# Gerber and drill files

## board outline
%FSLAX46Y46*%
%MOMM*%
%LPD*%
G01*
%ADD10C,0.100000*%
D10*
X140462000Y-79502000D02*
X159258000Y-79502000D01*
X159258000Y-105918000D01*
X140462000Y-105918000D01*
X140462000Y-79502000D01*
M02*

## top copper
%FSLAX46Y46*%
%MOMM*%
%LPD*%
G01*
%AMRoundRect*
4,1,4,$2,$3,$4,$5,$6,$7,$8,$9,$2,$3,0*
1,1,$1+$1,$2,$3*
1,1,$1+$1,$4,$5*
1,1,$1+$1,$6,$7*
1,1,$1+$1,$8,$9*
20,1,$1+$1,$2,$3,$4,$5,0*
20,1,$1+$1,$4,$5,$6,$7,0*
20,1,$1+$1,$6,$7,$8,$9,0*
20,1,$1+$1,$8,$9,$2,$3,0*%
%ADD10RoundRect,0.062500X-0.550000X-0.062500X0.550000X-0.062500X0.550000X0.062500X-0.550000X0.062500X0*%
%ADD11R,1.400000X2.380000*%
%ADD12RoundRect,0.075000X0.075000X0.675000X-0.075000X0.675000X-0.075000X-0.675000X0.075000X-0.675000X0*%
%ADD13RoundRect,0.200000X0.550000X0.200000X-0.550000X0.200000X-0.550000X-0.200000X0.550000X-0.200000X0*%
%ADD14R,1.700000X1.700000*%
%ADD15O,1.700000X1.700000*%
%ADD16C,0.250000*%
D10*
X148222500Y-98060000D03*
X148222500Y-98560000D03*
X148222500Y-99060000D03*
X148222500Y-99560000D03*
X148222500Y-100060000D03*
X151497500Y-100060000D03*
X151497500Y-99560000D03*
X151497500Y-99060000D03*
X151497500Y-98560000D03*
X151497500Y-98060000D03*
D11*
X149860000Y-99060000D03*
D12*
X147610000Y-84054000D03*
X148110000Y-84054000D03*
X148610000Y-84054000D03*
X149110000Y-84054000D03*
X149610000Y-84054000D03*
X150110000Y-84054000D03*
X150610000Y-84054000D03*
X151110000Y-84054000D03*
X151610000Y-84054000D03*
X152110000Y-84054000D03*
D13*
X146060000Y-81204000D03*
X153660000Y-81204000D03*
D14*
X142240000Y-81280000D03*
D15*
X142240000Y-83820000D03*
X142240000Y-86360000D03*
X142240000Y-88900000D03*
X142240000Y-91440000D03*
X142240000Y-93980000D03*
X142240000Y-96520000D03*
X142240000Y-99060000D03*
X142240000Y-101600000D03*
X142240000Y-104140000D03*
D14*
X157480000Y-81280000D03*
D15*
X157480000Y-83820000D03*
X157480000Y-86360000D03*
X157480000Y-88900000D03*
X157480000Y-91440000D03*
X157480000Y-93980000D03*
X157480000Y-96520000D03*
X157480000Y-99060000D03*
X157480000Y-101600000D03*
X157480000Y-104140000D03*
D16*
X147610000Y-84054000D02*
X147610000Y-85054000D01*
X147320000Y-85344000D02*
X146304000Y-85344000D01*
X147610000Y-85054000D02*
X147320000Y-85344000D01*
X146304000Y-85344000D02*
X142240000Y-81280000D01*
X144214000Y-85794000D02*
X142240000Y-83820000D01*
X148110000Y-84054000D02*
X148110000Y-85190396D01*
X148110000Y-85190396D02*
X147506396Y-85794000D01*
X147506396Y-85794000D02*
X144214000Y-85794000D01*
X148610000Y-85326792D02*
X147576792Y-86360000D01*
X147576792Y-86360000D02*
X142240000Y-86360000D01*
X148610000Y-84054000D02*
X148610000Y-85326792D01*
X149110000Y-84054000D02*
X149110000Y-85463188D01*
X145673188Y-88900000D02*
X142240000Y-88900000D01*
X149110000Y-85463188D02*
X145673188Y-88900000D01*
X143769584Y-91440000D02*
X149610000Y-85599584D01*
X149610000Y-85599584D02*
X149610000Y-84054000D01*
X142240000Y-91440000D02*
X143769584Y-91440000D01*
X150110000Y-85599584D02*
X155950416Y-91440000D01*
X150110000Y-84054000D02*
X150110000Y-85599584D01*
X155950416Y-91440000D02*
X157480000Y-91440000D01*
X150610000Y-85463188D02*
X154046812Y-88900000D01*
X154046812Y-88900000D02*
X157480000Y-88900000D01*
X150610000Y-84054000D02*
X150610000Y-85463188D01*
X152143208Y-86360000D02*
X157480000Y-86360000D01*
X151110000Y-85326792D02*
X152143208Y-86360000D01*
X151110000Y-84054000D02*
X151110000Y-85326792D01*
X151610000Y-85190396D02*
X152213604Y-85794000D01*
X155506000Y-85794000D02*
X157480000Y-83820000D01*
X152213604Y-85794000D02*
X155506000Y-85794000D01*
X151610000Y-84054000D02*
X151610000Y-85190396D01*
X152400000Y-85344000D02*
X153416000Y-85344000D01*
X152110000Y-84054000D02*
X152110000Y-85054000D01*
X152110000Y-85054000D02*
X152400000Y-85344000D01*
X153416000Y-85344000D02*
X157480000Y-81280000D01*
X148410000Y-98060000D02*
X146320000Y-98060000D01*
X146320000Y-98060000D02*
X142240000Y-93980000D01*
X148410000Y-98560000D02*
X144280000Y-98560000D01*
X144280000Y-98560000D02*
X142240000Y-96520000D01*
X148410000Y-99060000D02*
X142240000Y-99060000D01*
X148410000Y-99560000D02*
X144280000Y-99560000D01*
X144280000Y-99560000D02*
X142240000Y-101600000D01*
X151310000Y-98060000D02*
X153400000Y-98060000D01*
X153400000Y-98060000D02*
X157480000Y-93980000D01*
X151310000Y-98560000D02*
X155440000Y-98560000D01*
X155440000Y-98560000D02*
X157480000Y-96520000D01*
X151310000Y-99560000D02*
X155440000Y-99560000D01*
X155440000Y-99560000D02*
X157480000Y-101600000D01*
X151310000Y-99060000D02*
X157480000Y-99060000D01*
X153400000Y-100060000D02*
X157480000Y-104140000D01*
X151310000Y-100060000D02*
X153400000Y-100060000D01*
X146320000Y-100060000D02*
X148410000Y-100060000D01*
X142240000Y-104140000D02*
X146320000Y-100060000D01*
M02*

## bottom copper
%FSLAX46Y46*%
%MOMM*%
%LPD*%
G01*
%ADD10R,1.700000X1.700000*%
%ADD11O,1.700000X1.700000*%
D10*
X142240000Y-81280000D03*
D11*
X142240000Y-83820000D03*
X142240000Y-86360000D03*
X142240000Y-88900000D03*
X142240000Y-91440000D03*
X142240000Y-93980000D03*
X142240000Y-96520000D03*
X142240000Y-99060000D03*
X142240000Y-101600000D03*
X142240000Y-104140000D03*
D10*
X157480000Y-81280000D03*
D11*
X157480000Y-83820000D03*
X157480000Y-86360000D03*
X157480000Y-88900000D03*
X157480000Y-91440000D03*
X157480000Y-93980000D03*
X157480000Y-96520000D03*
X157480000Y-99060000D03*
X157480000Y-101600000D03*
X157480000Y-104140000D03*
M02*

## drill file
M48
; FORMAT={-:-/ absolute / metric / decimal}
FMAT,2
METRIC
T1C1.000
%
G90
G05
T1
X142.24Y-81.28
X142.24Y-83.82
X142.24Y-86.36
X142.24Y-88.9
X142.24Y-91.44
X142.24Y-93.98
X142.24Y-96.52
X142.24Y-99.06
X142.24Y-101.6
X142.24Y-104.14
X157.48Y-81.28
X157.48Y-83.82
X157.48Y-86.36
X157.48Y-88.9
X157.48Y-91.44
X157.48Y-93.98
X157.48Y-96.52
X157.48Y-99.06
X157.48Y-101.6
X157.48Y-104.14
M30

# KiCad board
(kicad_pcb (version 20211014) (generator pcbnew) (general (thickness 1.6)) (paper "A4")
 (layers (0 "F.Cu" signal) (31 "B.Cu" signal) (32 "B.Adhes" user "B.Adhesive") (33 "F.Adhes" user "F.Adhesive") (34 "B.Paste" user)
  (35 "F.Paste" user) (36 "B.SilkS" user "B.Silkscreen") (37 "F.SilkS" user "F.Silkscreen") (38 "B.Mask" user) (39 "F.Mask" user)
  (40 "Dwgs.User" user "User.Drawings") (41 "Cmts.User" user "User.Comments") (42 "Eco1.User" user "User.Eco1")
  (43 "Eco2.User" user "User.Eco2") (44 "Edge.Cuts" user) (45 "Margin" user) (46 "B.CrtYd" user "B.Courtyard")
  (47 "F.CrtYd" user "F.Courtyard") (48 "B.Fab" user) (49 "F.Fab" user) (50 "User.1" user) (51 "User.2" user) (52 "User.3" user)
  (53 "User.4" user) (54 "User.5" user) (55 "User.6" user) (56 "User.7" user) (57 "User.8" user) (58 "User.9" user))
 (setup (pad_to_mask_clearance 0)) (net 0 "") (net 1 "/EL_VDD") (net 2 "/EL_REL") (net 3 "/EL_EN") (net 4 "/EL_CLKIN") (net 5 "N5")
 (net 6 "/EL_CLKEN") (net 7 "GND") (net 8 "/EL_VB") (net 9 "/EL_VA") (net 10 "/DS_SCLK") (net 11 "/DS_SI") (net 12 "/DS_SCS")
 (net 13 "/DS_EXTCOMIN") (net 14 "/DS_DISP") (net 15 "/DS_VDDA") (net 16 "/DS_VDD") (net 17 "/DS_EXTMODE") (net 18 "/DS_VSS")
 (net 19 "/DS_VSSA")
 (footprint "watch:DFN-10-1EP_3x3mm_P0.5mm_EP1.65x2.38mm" (layer "F.Cu") (at 149.86 99.06)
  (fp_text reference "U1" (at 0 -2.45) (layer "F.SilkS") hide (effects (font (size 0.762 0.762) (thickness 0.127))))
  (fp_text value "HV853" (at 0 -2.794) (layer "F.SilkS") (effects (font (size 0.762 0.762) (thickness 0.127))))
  (pad "" smd roundrect (at -0.41 0.595) (size 0.67 0.96) (layers "F.Paste") (roundrect_rratio 0.25))
  (pad "" smd roundrect (at 0.41 0.595) (size 0.67 0.96) (layers "F.Paste") (roundrect_rratio 0.25))
  (pad "" smd roundrect (at 0.41 -0.595) (size 0.67 0.96) (layers "F.Paste") (roundrect_rratio 0.25))
  (pad "" smd roundrect (at -0.41 -0.595) (size 0.67 0.96) (layers "F.Paste") (roundrect_rratio 0.25))
  (pad "1" smd roundrect (at -1.6375 -1) (size 1.225 0.25) (layers "F.Cu" "F.Paste" "F.Mask") (roundrect_rratio 0.25) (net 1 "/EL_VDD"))
  (pad "2" smd roundrect (at -1.6375 -0.5) (size 1.225 0.25) (layers "F.Cu" "F.Paste" "F.Mask") (roundrect_rratio 0.25) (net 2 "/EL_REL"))
  (pad "3" smd roundrect (at -1.6375 0) (size 1.225 0.25) (layers "F.Cu" "F.Paste" "F.Mask") (roundrect_rratio 0.25) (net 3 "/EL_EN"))
  (pad "4" smd roundrect (at -1.6375 0.5) (size 1.225 0.25) (layers "F.Cu" "F.Paste" "F.Mask") (roundrect_rratio 0.25) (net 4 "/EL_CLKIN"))
  (pad "5" smd roundrect (at -1.6375 1) (size 1.225 0.25) (layers "F.Cu" "F.Paste" "F.Mask") (roundrect_rratio 0.25) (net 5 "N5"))
  (pad "6" smd roundrect (at 1.6375 1) (size 1.225 0.25) (layers "F.Cu" "F.Paste" "F.Mask") (roundrect_rratio 0.25) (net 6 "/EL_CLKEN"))
  (pad "7" smd roundrect (at 1.6375 0.5) (size 1.225 0.25) (layers "F.Cu" "F.Paste" "F.Mask") (roundrect_rratio 0.25) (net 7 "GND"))
  (pad "8" smd roundrect (at 1.6375 0) (size 1.225 0.25) (layers "F.Cu" "F.Paste" "F.Mask") (roundrect_rratio 0.25) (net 7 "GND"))
  (pad "9" smd roundrect (at 1.6375 -0.5) (size 1.225 0.25) (layers "F.Cu" "F.Paste" "F.Mask") (roundrect_rratio 0.25) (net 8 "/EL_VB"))
  (pad "10" smd roundrect (at 1.6375 -1) (size 1.225 0.25) (layers "F.Cu" "F.Paste" "F.Mask") (roundrect_rratio 0.25) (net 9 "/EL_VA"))
  (pad "11" smd rect (at 0 0) (size 1.4 2.38) (layers "F.Cu" "F.Mask")))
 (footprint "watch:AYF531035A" (layer "F.Cu") (at 149.86 81.204 180)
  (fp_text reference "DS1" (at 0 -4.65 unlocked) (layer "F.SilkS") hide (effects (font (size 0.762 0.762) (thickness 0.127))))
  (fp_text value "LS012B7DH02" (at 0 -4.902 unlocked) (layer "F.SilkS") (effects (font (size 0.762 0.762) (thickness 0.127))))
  (pad "1" smd roundrect (at 2.25 -2.85 180) (size 0.3 1.5) (layers "F.Cu" "F.Paste" "F.Mask") (roundrect_rratio 0.25) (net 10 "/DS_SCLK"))
  (pad "2" smd roundrect (at 1.75 -2.85 180) (size 0.3 1.5) (layers "F.Cu" "F.Paste" "F.Mask") (roundrect_rratio 0.25) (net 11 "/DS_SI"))
  (pad "3" smd roundrect (at 1.25 -2.85 180) (size 0.3 1.5) (layers "F.Cu" "F.Paste" "F.Mask") (roundrect_rratio 0.25) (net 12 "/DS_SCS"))
  (pad "4" smd roundrect (at 0.75 -2.85 180) (size 0.3 1.5) (layers "F.Cu" "F.Paste" "F.Mask") (roundrect_rratio 0.25)
   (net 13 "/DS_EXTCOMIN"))
  (pad "5" smd roundrect (at 0.25 -2.85 180) (size 0.3 1.5) (layers "F.Cu" "F.Paste" "F.Mask") (roundrect_rratio 0.25) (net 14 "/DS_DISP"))
  (pad "6" smd roundrect (at -0.25 -2.85 180) (size 0.3 1.5) (layers "F.Cu" "F.Paste" "F.Mask") (roundrect_rratio 0.25) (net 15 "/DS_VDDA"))
  (pad "7" smd roundrect (at -0.75 -2.85 180) (size 0.3 1.5) (layers "F.Cu" "F.Paste" "F.Mask") (roundrect_rratio 0.25) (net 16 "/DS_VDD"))
  (pad "8" smd roundrect (at -1.25 -2.85 180) (size 0.3 1.5) (layers "F.Cu" "F.Paste" "F.Mask") (roundrect_rratio 0.25)
   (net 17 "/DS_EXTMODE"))
  (pad "9" smd roundrect (at -1.75 -2.85 180) (size 0.3 1.5) (layers "F.Cu" "F.Paste" "F.Mask") (roundrect_rratio 0.25) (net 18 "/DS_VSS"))
  (pad "10" smd roundrect (at -2.25 -2.85 180) (size 0.3 1.5) (layers "F.Cu" "F.Paste" "F.Mask") (roundrect_rratio 0.25) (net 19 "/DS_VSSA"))
  (pad "MT" smd roundrect (at 3.8 0 180) (size 1.5 0.8) (layers "F.Cu" "F.Paste" "F.Mask") (roundrect_rratio 0.25))
  (pad "MT" smd roundrect (at -3.8 0 180) (size 1.5 0.8) (layers "F.Cu" "F.Paste" "F.Mask") (roundrect_rratio 0.25)))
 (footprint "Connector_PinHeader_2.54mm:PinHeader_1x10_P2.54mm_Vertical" (layer "B.Cu") (at 142.24 81.28 180)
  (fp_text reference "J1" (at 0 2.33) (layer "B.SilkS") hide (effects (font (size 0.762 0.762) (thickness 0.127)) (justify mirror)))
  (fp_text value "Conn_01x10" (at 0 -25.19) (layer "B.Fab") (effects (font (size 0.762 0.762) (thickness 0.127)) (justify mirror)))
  (pad "1" thru_hole rect (at 0 0 180) (size 1.7 1.7) (drill 1) (layers *.Cu *.Mask) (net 10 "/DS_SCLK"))
  (pad "2" thru_hole oval (at 0 -2.54 180) (size 1.7 1.7) (drill 1) (layers *.Cu *.Mask) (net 11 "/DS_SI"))
  (pad "3" thru_hole oval (at 0 -5.08 180) (size 1.7 1.7) (drill 1) (layers *.Cu *.Mask) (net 12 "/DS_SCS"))
  (pad "4" thru_hole oval (at 0 -7.62 180) (size 1.7 1.7) (drill 1) (layers *.Cu *.Mask) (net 13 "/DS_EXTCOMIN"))
  (pad "5" thru_hole oval (at 0 -10.16 180) (size 1.7 1.7) (drill 1) (layers *.Cu *.Mask) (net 14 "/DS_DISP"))
  (pad "6" thru_hole oval (at 0 -12.7 180) (size 1.7 1.7) (drill 1) (layers *.Cu *.Mask) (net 1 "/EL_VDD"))
  (pad "7" thru_hole oval (at 0 -15.24 180) (size 1.7 1.7) (drill 1) (layers *.Cu *.Mask) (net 2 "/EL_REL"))
  (pad "8" thru_hole oval (at 0 -17.78 180) (size 1.7 1.7) (drill 1) (layers *.Cu *.Mask) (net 3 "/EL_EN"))
  (pad "9" thru_hole oval (at 0 -20.32 180) (size 1.7 1.7) (drill 1) (layers *.Cu *.Mask) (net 4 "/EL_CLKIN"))
  (pad "10" thru_hole oval (at 0 -22.86 180) (size 1.7 1.7) (drill 1) (layers *.Cu *.Mask) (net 5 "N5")))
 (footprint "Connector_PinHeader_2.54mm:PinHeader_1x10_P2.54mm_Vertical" (layer "B.Cu") (at 157.48 81.28 180)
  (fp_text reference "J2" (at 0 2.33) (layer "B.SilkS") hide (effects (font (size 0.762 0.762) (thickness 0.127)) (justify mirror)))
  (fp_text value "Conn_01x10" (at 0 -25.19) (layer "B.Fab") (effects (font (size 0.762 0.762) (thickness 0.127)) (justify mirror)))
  (pad "1" thru_hole rect (at 0 0 180) (size 1.7 1.7) (drill 1) (layers *.Cu *.Mask) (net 19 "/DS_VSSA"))
  (pad "2" thru_hole oval (at 0 -2.54 180) (size 1.7 1.7) (drill 1) (layers *.Cu *.Mask) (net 18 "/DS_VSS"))
  (pad "3" thru_hole oval (at 0 -5.08 180) (size 1.7 1.7) (drill 1) (layers *.Cu *.Mask) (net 17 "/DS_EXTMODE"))
  (pad "4" thru_hole oval (at 0 -7.62 180) (size 1.7 1.7) (drill 1) (layers *.Cu *.Mask) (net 16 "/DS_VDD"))
  (pad "5" thru_hole oval (at 0 -10.16 180) (size 1.7 1.7) (drill 1) (layers *.Cu *.Mask) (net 15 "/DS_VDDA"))
  (pad "6" thru_hole oval (at 0 -12.7 180) (size 1.7 1.7) (drill 1) (layers *.Cu *.Mask) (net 9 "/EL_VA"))
  (pad "7" thru_hole oval (at 0 -15.24 180) (size 1.7 1.7) (drill 1) (layers *.Cu *.Mask) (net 8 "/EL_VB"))
  (pad "8" thru_hole oval (at 0 -17.78 180) (size 1.7 1.7) (drill 1) (layers *.Cu *.Mask) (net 7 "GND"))
  (pad "9" thru_hole oval (at 0 -20.32 180) (size 1.7 1.7) (drill 1) (layers *.Cu *.Mask) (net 7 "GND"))
  (pad "10" thru_hole oval (at 0 -22.86 180) (size 1.7 1.7) (drill 1) (layers *.Cu *.Mask) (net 6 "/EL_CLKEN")))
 (gr_rect (start 140.462 79.502) (end 159.258 105.918) (layer "Edge.Cuts") (width 0.1) (fill none))
 (segment (start 147.61 84.054) (end 147.61 85.054) (width 0.25) (layer "F.Cu") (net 10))
 (segment (start 147.32 85.344) (end 146.304 85.344) (width 0.25) (layer "F.Cu") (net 10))
 (segment (start 147.61 85.054) (end 147.32 85.344) (width 0.25) (layer "F.Cu") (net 10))
 (segment (start 146.304 85.344) (end 142.24 81.28) (width 0.25) (layer "F.Cu") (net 10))
 (segment (start 144.214 85.794) (end 142.24 83.82) (width 0.25) (layer "F.Cu") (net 11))
 (segment (start 148.11 84.054) (end 148.11 85.190396) (width 0.25) (layer "F.Cu") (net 11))
 (segment (start 148.11 85.190396) (end 147.506396 85.794) (width 0.25) (layer "F.Cu") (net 11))
 (segment (start 147.506396 85.794) (end 144.214 85.794) (width 0.25) (layer "F.Cu") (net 11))
 (segment (start 148.61 85.326792) (end 147.576792 86.36) (width 0.25) (layer "F.Cu") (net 12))
 (segment (start 147.576792 86.36) (end 142.24 86.36) (width 0.25) (layer "F.Cu") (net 12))
 (segment (start 148.61 84.054) (end 148.61 85.326792) (width 0.25) (layer "F.Cu") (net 12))
 (segment (start 149.11 84.054) (end 149.11 85.463188) (width 0.25) (layer "F.Cu") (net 13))
 (segment (start 145.673188 88.9) (end 142.24 88.9) (width 0.25) (layer "F.Cu") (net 13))
 (segment (start 149.11 85.463188) (end 145.673188 88.9) (width 0.25) (layer "F.Cu") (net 13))
 (segment (start 143.769584 91.44) (end 149.61 85.599584) (width 0.25) (layer "F.Cu") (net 14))
 (segment (start 149.61 85.599584) (end 149.61 84.054) (width 0.25) (layer "F.Cu") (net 14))
 (segment (start 142.24 91.44) (end 143.769584 91.44) (width 0.25) (layer "F.Cu") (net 14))
 (segment (start 150.11 85.599584) (end 155.950416 91.44) (width 0.25) (layer "F.Cu") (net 15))
 (segment (start 150.11 84.054) (end 150.11 85.599584) (width 0.25) (layer "F.Cu") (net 15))
 (segment (start 155.950416 91.44) (end 157.48 91.44) (width 0.25) (layer "F.Cu") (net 15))
 (segment (start 150.61 85.463188) (end 154.046812 88.9) (width 0.25) (layer "F.Cu") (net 16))
 (segment (start 154.046812 88.9) (end 157.48 88.9) (width 0.25) (layer "F.Cu") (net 16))
 (segment (start 150.61 84.054) (end 150.61 85.463188) (width 0.25) (layer "F.Cu") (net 16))
 (segment (start 152.143208 86.36) (end 157.48 86.36) (width 0.25) (layer "F.Cu") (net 17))
 (segment (start 151.11 85.326792) (end 152.143208 86.36) (width 0.25) (layer "F.Cu") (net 17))
 (segment (start 151.11 84.054) (end 151.11 85.326792) (width 0.25) (layer "F.Cu") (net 17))
 (segment (start 151.61 85.190396) (end 152.213604 85.794) (width 0.25) (layer "F.Cu") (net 18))
 (segment (start 155.506 85.794) (end 157.48 83.82) (width 0.25) (layer "F.Cu") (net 18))
 (segment (start 152.213604 85.794) (end 155.506 85.794) (width 0.25) (layer "F.Cu") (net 18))
 (segment (start 151.61 84.054) (end 151.61 85.190396) (width 0.25) (layer "F.Cu") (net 18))
 (segment (start 152.4 85.344) (end 153.416 85.344) (width 0.25) (layer "F.Cu") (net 19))
 (segment (start 152.11 84.054) (end 152.11 85.054) (width 0.25) (layer "F.Cu") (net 19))
 (segment (start 152.11 85.054) (end 152.4 85.344) (width 0.25) (layer "F.Cu") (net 19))
 (segment (start 153.416 85.344) (end 157.48 81.28) (width 0.25) (layer "F.Cu") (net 19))
 (segment (start 148.41 98.06) (end 146.32 98.06) (width 0.25) (layer "F.Cu") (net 1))
 (segment (start 146.32 98.06) (end 142.24 93.98) (width 0.25) (layer "F.Cu") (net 1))
 (segment (start 148.41 98.56) (end 144.28 98.56) (width 0.25) (layer "F.Cu") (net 2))
 (segment (start 144.28 98.56) (end 142.24 96.52) (width 0.25) (layer "F.Cu") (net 2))
 (segment (start 148.41 99.06) (end 142.24 99.06) (width 0.25) (layer "F.Cu") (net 3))
 (segment (start 148.41 99.56) (end 144.28 99.56) (width 0.25) (layer "F.Cu") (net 4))
 (segment (start 144.28 99.56) (end 142.24 101.6) (width 0.25) (layer "F.Cu") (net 4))
 (segment (start 151.31 98.06) (end 153.4 98.06) (width 0.25) (layer "F.Cu") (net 9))
 (segment (start 153.4 98.06) (end 157.48 93.98) (width 0.25) (layer "F.Cu") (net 9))
 (segment (start 151.31 98.56) (end 155.44 98.56) (width 0.25) (layer "F.Cu") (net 8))
 (segment (start 155.44 98.56) (end 157.48 96.52) (width 0.25) (layer "F.Cu") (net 8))
 (segment (start 151.31 99.56) (end 155.44 99.56) (width 0.25) (layer "F.Cu") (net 7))
 (segment (start 155.44 99.56) (end 157.48 101.6) (width 0.25) (layer "F.Cu") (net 7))
 (segment (start 151.31 99.06) (end 157.48 99.06) (width 0.25) (layer "F.Cu") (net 7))
 (segment (start 153.4 100.06) (end 157.48 104.14) (width 0.25) (layer "F.Cu") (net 6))
 (segment (start 151.31 100.06) (end 153.4 100.06) (width 0.25) (layer "F.Cu") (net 6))
 (segment (start 146.32 100.06) (end 148.41 100.06) (width 0.25) (layer "F.Cu") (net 5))
 (segment (start 142.24 104.14) (end 146.32 100.06) (width 0.25) (layer "F.Cu") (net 5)))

